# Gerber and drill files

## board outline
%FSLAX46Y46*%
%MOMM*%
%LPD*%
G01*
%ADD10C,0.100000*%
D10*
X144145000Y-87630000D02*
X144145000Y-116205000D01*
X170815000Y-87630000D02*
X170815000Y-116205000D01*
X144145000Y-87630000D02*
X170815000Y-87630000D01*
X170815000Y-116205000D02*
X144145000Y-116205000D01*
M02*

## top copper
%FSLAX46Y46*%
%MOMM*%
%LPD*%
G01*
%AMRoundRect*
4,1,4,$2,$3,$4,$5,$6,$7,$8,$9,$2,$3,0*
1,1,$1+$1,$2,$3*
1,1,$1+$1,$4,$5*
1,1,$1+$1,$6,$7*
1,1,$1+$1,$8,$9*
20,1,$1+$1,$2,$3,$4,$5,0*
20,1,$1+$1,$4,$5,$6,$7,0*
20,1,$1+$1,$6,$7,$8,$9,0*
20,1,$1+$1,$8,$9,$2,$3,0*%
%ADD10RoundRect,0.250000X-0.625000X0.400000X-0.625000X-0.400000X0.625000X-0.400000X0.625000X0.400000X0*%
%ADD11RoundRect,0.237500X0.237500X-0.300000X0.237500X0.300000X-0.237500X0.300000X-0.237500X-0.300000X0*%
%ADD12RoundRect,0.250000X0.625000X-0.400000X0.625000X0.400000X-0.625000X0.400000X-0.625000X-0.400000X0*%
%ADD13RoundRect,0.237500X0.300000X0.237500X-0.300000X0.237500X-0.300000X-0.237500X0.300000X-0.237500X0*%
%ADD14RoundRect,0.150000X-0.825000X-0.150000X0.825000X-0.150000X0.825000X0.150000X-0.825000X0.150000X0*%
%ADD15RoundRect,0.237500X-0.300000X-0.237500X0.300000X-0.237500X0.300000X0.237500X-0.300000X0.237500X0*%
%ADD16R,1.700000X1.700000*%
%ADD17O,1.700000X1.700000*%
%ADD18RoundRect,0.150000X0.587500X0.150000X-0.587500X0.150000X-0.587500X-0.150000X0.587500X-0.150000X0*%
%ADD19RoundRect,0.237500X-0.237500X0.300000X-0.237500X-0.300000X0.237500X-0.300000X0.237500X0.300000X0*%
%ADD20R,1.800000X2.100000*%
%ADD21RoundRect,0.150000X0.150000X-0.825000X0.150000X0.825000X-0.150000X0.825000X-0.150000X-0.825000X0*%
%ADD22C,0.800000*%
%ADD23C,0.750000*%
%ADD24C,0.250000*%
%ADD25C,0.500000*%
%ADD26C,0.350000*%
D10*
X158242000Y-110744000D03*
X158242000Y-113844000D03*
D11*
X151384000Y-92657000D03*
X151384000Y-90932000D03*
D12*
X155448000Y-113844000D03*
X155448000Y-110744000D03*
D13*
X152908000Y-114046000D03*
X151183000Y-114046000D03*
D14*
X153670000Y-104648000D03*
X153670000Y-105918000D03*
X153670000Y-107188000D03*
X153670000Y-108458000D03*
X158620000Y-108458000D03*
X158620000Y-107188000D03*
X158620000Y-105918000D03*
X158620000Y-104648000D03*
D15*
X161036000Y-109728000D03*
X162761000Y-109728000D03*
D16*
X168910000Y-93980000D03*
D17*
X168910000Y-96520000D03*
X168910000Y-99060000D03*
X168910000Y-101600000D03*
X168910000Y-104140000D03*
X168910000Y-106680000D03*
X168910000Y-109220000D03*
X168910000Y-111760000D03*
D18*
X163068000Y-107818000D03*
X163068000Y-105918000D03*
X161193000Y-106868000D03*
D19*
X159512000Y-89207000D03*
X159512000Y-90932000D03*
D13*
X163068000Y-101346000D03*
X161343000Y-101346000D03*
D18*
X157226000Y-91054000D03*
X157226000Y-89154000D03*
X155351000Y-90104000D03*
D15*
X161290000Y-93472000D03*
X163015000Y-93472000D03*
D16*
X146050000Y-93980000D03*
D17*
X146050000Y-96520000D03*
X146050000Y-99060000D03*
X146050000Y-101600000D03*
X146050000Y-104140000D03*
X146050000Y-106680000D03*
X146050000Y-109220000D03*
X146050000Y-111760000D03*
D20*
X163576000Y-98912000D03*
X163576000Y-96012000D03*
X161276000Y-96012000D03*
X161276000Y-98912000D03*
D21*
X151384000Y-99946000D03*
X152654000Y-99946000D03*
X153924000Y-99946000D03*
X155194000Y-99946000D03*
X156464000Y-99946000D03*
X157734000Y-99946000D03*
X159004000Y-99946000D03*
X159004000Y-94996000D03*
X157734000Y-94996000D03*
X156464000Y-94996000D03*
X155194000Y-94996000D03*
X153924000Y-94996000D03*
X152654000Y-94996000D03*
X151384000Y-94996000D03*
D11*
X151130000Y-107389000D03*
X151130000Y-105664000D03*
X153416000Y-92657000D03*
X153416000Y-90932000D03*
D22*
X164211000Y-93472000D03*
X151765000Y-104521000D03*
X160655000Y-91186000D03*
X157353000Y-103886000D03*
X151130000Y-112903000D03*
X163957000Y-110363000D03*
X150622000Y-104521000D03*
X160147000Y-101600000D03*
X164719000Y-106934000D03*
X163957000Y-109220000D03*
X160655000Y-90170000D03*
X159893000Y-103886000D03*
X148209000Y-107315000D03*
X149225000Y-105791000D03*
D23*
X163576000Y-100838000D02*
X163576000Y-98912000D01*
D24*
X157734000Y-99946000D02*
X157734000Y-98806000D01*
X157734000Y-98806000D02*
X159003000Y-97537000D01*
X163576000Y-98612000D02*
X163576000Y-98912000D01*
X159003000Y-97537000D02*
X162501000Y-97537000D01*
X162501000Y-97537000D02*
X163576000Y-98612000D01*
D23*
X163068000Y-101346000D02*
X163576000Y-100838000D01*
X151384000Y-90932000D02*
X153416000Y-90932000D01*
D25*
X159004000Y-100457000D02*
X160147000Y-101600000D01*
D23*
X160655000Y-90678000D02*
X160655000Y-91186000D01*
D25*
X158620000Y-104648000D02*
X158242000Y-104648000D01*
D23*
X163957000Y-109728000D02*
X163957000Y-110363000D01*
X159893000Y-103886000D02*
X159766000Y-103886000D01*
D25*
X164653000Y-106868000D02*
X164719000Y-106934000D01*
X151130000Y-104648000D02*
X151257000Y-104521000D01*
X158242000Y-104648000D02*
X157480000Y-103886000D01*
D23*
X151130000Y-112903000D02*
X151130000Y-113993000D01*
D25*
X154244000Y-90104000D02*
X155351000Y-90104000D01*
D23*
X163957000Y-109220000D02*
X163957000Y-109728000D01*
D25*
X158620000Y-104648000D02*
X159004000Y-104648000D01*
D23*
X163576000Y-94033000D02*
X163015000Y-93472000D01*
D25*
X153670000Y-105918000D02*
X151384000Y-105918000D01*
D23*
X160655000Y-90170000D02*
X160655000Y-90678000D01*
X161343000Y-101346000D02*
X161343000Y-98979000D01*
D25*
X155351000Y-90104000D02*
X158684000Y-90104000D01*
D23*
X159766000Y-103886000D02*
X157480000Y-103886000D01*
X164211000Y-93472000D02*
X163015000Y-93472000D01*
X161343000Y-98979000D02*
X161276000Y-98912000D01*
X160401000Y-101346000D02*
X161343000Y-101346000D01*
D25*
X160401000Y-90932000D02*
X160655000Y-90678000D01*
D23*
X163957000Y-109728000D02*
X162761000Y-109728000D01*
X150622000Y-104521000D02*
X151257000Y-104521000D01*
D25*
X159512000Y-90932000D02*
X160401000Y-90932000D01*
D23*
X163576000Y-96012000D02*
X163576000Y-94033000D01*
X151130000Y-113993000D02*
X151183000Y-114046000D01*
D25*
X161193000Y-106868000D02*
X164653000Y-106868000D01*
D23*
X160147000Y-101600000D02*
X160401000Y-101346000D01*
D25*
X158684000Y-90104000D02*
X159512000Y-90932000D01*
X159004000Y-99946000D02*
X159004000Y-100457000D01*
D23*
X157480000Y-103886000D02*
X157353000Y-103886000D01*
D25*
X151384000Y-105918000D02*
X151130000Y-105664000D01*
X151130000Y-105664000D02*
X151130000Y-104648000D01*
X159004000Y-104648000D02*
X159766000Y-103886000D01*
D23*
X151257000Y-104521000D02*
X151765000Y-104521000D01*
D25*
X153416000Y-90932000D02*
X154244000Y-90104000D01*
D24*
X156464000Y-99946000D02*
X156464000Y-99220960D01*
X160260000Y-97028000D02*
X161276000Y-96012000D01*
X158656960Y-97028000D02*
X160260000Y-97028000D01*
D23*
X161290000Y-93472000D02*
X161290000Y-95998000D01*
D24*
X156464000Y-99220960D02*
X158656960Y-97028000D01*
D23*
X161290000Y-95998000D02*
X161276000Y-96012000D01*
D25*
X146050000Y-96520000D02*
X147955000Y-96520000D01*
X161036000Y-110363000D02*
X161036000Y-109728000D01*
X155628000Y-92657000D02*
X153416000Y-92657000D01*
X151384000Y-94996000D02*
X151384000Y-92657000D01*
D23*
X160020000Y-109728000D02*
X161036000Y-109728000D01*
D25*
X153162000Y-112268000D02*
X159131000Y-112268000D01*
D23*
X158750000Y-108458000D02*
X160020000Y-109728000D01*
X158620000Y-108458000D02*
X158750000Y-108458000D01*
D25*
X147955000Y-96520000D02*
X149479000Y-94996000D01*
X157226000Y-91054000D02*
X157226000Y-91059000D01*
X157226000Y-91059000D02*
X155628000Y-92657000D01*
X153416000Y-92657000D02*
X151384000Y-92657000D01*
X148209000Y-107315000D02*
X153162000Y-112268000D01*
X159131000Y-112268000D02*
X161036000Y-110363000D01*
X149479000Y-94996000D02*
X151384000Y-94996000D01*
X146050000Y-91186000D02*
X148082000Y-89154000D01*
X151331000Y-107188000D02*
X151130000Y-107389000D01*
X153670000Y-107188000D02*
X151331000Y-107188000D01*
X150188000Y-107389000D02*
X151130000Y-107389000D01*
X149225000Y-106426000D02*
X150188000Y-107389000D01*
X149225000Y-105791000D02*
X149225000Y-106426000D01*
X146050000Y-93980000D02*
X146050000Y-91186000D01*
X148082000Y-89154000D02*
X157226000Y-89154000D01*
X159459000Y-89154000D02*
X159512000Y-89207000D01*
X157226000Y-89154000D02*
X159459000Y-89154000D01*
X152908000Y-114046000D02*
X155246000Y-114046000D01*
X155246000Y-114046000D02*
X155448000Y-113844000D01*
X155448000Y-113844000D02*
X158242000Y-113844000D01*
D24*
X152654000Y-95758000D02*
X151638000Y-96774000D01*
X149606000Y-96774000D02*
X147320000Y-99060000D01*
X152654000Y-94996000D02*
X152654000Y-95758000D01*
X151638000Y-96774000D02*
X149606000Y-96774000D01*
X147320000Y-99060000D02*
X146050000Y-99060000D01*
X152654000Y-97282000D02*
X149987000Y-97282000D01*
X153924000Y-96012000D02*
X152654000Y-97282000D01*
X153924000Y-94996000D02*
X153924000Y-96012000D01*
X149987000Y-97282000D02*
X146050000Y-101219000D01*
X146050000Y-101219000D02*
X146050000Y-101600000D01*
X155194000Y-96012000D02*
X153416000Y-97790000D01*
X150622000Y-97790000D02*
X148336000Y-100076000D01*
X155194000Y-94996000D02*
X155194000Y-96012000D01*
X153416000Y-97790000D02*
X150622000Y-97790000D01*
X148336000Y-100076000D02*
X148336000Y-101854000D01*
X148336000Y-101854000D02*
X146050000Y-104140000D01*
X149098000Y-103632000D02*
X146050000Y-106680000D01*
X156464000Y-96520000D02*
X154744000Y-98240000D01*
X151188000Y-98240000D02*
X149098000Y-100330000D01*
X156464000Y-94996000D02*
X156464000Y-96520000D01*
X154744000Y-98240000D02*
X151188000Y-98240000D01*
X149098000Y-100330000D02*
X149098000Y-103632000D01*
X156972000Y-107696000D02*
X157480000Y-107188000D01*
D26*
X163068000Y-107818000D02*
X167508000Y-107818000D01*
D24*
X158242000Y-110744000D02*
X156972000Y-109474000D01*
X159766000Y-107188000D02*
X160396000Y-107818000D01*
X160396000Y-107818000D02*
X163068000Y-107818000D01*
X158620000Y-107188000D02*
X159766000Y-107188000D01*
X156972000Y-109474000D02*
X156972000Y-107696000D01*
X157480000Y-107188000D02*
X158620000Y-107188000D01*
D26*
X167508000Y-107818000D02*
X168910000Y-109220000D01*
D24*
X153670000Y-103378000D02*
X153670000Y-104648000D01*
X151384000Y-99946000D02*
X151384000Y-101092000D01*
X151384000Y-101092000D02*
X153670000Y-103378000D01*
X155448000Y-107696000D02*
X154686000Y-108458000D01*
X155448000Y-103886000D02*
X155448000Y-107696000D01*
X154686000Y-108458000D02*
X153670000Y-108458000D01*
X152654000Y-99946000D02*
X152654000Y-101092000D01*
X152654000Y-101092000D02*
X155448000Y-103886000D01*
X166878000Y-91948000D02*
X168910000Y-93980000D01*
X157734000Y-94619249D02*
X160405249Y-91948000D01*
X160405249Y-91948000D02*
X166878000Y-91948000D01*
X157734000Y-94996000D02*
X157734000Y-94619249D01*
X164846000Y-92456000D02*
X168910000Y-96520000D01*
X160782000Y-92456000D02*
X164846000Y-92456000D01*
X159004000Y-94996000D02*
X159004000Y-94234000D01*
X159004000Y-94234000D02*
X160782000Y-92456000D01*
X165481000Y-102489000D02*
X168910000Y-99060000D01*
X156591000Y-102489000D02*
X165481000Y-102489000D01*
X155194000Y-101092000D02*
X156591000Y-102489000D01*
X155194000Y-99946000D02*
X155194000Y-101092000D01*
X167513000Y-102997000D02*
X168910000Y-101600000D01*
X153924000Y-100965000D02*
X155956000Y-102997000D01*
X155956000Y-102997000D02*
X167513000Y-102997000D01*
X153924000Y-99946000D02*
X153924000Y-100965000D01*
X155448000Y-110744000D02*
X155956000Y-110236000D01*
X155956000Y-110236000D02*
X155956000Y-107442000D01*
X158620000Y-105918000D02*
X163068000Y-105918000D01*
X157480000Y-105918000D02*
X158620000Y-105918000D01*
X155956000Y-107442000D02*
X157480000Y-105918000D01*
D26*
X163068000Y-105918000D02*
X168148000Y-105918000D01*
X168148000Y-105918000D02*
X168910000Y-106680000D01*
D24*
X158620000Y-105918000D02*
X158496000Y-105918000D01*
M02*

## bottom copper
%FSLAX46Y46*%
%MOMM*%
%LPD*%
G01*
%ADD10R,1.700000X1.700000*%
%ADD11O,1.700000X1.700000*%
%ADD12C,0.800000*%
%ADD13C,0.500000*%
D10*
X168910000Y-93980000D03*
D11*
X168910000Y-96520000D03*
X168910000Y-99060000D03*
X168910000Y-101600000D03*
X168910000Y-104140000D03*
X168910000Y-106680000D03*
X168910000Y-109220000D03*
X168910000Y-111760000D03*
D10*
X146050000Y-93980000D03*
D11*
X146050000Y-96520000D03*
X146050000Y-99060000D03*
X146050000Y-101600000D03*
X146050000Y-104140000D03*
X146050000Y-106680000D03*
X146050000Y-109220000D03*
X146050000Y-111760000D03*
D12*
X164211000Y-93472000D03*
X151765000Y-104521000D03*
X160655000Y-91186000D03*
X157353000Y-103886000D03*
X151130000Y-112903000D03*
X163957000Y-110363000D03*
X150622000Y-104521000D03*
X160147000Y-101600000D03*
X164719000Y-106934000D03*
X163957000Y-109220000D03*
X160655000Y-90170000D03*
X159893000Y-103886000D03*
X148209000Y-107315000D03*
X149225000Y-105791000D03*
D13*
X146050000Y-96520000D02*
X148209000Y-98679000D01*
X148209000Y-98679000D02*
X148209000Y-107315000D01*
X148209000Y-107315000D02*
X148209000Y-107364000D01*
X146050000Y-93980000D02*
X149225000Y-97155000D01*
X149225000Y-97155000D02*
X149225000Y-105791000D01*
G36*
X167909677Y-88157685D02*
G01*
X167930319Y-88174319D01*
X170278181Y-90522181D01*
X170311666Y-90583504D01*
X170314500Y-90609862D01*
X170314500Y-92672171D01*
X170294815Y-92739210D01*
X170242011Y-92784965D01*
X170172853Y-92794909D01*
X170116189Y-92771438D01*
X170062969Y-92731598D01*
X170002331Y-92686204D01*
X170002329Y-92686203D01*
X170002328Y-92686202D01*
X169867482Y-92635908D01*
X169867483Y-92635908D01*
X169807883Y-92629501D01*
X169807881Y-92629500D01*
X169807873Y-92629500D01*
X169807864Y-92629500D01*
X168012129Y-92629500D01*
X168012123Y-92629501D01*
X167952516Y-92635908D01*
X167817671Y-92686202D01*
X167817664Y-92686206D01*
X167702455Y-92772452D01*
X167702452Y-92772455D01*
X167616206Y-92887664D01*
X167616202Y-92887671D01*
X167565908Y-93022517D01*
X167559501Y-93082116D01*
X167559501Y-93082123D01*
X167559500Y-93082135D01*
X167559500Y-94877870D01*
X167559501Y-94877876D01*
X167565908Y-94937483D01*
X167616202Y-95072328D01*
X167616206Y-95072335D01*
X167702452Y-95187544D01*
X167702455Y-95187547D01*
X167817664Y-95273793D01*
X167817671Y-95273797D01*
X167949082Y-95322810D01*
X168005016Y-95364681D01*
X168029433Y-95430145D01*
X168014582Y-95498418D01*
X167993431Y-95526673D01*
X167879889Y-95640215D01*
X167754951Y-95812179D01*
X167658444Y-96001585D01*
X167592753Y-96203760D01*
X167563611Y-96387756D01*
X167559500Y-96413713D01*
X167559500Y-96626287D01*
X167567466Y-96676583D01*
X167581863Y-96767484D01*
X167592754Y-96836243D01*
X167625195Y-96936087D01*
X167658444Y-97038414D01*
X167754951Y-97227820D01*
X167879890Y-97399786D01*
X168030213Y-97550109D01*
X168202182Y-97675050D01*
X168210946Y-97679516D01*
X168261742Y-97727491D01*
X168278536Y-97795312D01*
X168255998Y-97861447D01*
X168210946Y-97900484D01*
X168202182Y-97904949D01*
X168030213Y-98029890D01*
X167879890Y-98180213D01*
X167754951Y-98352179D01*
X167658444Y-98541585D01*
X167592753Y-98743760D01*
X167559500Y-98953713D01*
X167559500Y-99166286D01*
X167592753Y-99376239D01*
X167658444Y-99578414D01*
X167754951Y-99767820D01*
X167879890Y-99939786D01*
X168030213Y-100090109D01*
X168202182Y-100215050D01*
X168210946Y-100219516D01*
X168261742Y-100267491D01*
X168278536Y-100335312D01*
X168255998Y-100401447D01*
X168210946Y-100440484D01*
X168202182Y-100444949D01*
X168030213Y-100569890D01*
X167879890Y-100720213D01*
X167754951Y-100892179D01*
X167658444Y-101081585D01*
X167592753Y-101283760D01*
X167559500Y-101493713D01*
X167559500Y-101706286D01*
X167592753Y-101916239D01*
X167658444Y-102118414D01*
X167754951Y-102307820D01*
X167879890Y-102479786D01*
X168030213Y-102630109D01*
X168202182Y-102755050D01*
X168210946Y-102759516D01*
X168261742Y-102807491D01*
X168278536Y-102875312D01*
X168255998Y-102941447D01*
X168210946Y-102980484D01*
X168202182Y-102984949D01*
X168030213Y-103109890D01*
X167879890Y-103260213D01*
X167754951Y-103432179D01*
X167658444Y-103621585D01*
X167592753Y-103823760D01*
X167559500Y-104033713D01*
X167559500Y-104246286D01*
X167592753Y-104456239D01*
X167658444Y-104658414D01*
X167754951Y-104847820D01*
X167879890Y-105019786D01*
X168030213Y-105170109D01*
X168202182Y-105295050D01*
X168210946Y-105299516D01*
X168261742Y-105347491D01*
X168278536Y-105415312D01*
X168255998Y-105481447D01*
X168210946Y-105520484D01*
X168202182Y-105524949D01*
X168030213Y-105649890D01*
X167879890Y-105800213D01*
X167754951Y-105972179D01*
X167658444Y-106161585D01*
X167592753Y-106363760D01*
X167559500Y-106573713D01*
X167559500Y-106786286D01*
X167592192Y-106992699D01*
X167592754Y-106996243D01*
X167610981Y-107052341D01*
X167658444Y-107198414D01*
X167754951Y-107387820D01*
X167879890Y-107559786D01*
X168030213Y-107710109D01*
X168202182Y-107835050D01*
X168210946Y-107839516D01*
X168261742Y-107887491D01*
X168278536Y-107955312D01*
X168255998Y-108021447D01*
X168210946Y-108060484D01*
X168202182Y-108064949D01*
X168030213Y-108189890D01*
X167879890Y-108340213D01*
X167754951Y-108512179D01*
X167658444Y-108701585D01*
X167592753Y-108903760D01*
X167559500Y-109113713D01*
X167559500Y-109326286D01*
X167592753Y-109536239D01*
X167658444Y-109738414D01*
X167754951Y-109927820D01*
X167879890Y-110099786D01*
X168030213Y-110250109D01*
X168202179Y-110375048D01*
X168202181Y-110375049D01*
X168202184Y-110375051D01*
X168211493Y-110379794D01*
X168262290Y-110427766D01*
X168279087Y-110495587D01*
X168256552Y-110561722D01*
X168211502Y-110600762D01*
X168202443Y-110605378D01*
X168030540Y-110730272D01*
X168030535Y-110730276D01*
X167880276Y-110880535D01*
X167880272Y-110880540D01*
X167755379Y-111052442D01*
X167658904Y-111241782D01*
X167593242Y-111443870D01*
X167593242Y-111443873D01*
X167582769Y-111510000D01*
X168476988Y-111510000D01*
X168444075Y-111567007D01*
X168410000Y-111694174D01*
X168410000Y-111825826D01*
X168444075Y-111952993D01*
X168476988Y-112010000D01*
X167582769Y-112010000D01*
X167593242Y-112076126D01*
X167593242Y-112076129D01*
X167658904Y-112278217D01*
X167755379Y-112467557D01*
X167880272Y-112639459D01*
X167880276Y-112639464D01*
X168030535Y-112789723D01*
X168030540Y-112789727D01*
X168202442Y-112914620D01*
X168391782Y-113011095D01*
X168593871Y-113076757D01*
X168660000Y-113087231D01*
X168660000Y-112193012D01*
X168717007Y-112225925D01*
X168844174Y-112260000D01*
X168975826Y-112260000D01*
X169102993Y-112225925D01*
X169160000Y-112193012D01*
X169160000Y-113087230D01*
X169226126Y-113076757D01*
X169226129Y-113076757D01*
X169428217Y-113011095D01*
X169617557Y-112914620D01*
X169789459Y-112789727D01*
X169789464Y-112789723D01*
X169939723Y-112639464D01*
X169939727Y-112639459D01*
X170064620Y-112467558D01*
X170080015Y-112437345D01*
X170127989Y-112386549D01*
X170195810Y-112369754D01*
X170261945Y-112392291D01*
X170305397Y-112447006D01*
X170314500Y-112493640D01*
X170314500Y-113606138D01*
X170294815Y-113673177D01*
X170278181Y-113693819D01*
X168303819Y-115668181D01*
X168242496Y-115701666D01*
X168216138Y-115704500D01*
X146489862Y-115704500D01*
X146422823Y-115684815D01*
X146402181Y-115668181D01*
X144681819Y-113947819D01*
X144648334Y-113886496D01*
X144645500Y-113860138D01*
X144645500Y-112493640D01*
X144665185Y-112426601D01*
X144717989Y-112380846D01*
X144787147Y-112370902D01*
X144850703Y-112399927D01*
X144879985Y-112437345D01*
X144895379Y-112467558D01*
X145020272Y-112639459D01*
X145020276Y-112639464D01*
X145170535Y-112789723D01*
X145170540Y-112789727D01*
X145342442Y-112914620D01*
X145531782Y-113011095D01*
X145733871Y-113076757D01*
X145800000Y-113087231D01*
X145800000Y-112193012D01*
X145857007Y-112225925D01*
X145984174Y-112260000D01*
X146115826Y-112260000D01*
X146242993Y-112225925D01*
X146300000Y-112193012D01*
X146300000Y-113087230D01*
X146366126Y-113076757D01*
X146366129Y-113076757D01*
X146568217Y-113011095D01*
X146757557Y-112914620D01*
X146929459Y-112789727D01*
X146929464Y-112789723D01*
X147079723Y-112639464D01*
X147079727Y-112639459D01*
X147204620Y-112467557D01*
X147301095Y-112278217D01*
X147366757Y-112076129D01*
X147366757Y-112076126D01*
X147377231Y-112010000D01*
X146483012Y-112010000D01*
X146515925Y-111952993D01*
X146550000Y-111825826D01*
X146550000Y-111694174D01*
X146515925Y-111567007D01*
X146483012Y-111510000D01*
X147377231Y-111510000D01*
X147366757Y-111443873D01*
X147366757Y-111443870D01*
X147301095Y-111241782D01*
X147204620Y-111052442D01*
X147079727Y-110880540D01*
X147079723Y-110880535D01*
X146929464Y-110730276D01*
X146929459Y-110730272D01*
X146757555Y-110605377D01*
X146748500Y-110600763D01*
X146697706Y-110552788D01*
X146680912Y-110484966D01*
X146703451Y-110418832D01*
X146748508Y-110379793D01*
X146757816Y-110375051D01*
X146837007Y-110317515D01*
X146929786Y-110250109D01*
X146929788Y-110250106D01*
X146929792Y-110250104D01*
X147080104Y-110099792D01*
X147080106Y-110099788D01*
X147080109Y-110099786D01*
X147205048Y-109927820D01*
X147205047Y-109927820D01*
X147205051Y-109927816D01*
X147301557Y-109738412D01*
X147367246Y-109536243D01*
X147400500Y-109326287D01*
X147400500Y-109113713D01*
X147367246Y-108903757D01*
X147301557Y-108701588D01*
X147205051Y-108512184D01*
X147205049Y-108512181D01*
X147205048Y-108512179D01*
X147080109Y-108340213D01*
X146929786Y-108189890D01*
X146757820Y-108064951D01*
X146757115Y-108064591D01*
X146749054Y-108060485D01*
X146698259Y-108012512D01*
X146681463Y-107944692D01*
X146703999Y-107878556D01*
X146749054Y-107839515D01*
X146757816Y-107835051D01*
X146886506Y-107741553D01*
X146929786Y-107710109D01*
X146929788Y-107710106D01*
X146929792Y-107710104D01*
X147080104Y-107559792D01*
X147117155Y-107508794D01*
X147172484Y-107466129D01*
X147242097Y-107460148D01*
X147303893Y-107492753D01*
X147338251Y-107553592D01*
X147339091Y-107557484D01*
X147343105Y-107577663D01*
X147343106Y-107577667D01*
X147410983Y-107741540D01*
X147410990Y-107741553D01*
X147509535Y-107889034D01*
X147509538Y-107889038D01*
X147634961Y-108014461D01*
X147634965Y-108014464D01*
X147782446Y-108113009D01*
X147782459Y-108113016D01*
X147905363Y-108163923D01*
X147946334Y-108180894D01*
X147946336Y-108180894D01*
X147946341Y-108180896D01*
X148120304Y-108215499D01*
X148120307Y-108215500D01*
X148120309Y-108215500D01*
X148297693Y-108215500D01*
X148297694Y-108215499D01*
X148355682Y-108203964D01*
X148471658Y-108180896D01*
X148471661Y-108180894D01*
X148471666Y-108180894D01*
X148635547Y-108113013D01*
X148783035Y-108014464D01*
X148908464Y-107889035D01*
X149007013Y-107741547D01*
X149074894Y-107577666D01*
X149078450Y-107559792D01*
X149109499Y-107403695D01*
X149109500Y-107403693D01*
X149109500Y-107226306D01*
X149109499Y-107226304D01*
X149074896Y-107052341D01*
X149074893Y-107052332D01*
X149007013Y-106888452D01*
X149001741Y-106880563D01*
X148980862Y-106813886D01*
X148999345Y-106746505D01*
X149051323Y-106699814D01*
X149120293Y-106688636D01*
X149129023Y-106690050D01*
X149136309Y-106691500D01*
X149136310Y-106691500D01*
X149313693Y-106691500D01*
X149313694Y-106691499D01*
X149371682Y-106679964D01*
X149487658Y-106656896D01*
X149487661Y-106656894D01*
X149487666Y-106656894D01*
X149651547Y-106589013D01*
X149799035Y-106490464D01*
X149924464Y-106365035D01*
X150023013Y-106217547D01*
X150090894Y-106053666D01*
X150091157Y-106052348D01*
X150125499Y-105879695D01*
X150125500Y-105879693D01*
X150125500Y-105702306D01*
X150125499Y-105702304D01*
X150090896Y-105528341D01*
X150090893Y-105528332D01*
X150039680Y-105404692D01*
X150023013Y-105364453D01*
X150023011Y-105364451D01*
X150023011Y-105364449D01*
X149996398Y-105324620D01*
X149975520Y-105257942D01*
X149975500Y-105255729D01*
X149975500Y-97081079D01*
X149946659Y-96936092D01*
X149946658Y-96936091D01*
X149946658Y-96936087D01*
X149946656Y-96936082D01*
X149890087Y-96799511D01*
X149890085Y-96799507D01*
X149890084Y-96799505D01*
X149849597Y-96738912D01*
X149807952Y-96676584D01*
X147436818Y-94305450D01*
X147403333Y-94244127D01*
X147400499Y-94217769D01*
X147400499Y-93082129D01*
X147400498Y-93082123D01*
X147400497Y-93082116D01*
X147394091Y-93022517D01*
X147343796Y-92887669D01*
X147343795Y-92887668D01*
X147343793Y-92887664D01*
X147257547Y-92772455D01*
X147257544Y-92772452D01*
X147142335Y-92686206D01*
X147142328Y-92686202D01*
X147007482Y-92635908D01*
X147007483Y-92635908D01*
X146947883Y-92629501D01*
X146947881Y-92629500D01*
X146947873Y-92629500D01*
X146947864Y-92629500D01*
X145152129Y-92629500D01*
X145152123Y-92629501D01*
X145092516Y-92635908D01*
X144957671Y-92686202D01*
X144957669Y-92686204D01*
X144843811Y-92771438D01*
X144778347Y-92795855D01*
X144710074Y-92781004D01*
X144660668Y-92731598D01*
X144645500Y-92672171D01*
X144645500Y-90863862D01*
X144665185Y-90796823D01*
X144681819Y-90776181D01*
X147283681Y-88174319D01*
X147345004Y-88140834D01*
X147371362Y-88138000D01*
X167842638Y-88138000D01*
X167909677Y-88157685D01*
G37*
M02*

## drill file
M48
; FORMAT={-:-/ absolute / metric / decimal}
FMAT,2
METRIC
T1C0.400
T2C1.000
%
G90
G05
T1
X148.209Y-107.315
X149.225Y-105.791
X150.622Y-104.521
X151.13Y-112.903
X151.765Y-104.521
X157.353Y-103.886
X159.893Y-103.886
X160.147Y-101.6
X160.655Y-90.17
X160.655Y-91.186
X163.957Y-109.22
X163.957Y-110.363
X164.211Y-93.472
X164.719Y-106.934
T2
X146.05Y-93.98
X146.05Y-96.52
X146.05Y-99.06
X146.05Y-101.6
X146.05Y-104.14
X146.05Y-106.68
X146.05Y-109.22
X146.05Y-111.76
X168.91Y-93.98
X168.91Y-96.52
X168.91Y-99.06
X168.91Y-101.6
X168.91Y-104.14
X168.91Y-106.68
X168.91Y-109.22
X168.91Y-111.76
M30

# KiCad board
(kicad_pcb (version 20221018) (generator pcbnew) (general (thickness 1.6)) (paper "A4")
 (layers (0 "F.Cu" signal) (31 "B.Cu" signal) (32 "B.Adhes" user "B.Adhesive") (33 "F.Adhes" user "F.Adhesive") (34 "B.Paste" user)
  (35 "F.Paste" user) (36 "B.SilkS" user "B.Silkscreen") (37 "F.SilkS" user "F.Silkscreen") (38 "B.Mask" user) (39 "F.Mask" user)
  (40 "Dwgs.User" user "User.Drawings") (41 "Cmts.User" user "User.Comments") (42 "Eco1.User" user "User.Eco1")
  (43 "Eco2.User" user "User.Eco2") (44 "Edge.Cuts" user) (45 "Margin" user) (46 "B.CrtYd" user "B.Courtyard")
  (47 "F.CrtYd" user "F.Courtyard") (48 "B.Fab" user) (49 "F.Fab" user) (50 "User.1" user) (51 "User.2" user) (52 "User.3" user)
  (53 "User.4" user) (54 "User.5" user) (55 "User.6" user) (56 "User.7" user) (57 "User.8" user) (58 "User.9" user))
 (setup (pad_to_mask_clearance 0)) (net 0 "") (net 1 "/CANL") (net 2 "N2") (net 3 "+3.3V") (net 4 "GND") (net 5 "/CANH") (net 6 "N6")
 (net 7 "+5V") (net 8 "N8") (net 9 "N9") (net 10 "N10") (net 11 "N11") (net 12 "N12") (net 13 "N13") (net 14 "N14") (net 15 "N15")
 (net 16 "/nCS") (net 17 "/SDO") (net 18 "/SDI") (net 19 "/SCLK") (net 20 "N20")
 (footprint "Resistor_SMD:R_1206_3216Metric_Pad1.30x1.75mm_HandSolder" (layer "F.Cu") (at 158.242 112.294 -90)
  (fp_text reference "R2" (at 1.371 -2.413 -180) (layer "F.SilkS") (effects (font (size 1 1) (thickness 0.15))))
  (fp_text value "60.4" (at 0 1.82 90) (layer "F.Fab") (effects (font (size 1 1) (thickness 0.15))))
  (pad "1" smd roundrect (at -1.55 0 270) (size 1.3 1.75) (layers "F.Cu" "F.Paste" "F.Mask") (roundrect_rratio 0.1923076923) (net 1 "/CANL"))
  (pad "2" smd roundrect (at 1.55 0 270) (size 1.3 1.75) (layers "F.Cu" "F.Paste" "F.Mask") (roundrect_rratio 0.1923076923) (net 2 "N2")))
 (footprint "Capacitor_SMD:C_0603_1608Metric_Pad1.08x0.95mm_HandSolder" (layer "F.Cu") (at 151.384 91.7945 90)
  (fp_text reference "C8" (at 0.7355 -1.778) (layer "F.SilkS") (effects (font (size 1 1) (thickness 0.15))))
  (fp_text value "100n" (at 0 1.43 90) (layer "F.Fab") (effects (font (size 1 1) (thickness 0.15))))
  (pad "1" smd roundrect (at -0.8625 0 90) (size 1.075 0.95) (layers "F.Cu" "F.Paste" "F.Mask") (roundrect_rratio 0.25) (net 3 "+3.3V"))
  (pad "2" smd roundrect (at 0.8625 0 90) (size 1.075 0.95) (layers "F.Cu" "F.Paste" "F.Mask") (roundrect_rratio 0.25) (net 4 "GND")))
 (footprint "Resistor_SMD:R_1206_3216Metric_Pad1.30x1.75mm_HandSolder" (layer "F.Cu") (at 155.448 112.294 90)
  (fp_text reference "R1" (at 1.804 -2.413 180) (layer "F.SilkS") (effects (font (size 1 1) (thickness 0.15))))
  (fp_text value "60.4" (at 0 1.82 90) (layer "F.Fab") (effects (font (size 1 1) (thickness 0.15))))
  (pad "1" smd roundrect (at -1.55 0 90) (size 1.3 1.75) (layers "F.Cu" "F.Paste" "F.Mask") (roundrect_rratio 0.1923076923) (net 2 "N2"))
  (pad "2" smd roundrect (at 1.55 0 90) (size 1.3 1.75) (layers "F.Cu" "F.Paste" "F.Mask") (roundrect_rratio 0.1923076923) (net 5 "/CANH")))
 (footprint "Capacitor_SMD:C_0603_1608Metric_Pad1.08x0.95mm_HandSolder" (layer "F.Cu") (at 152.0455 114.046 180)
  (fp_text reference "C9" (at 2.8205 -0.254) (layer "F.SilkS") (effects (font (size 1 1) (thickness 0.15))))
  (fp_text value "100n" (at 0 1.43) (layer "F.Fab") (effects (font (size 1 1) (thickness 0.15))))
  (pad "1" smd roundrect (at -0.8625 0 180) (size 1.075 0.95) (layers "F.Cu" "F.Paste" "F.Mask") (roundrect_rratio 0.25) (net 2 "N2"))
  (pad "2" smd roundrect (at 0.8625 0 180) (size 1.075 0.95) (layers "F.Cu" "F.Paste" "F.Mask") (roundrect_rratio 0.25) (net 4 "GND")))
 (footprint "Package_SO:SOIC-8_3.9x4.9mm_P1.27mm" (layer "F.Cu") (at 156.145 106.553)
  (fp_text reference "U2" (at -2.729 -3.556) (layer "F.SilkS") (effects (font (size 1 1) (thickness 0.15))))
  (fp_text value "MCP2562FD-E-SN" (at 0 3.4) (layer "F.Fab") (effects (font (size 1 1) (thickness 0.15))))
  (pad "1" smd roundrect (at -2.475 -1.905) (size 1.95 0.6) (layers "F.Cu" "F.Paste" "F.Mask") (roundrect_rratio 0.25) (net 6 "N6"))
  (pad "2" smd roundrect (at -2.475 -0.635) (size 1.95 0.6) (layers "F.Cu" "F.Paste" "F.Mask") (roundrect_rratio 0.25) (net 4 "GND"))
  (pad "3" smd roundrect (at -2.475 0.635) (size 1.95 0.6) (layers "F.Cu" "F.Paste" "F.Mask") (roundrect_rratio 0.25) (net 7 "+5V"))
  (pad "4" smd roundrect (at -2.475 1.905) (size 1.95 0.6) (layers "F.Cu" "F.Paste" "F.Mask") (roundrect_rratio 0.25) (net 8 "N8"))
  (pad "5" smd roundrect (at 2.475 1.905) (size 1.95 0.6) (layers "F.Cu" "F.Paste" "F.Mask") (roundrect_rratio 0.25) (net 3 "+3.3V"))
  (pad "6" smd roundrect (at 2.475 0.635) (size 1.95 0.6) (layers "F.Cu" "F.Paste" "F.Mask") (roundrect_rratio 0.25) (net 1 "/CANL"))
  (pad "7" smd roundrect (at 2.475 -0.635) (size 1.95 0.6) (layers "F.Cu" "F.Paste" "F.Mask") (roundrect_rratio 0.25) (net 5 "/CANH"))
  (pad "8" smd roundrect (at 2.475 -1.905) (size 1.95 0.6) (layers "F.Cu" "F.Paste" "F.Mask") (roundrect_rratio 0.25) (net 4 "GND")))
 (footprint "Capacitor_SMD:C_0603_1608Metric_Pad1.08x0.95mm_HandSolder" (layer "F.Cu") (at 161.8985 109.728)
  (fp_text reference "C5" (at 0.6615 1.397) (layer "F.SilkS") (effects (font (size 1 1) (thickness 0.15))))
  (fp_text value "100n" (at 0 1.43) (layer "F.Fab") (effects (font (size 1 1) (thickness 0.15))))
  (pad "1" smd roundrect (at -0.8625 0) (size 1.075 0.95) (layers "F.Cu" "F.Paste" "F.Mask") (roundrect_rratio 0.25) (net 3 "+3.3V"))
  (pad "2" smd roundrect (at 0.8625 0) (size 1.075 0.95) (layers "F.Cu" "F.Paste" "F.Mask") (roundrect_rratio 0.25) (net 4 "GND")))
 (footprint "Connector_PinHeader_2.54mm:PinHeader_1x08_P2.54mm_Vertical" (layer "F.Cu") (at 168.91 93.98)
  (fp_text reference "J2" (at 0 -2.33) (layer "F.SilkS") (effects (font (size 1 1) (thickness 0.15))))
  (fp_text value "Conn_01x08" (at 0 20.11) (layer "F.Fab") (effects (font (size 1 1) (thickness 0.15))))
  (pad "1" thru_hole rect (at 0 0) (size 1.7 1.7) (drill 1) (layers "*.Cu" "*.Mask") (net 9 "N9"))
  (pad "2" thru_hole oval (at 0 2.54) (size 1.7 1.7) (drill 1) (layers "*.Cu" "*.Mask") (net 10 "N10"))
  (pad "3" thru_hole oval (at 0 5.08) (size 1.7 1.7) (drill 1) (layers "*.Cu" "*.Mask") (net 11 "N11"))
  (pad "4" thru_hole oval (at 0 7.62) (size 1.7 1.7) (drill 1) (layers "*.Cu" "*.Mask") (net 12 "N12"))
  (pad "5" thru_hole oval (at 0 10.16) (size 1.7 1.7) (drill 1) (layers "*.Cu" "*.Mask") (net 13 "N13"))
  (pad "6" thru_hole oval (at 0 12.7) (size 1.7 1.7) (drill 1) (layers "*.Cu" "*.Mask") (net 5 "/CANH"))
  (pad "7" thru_hole oval (at 0 15.24) (size 1.7 1.7) (drill 1) (layers "*.Cu" "*.Mask") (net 1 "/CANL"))
  (pad "8" thru_hole oval (at 0 17.78) (size 1.7 1.7) (drill 1) (layers "*.Cu" "*.Mask") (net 4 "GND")))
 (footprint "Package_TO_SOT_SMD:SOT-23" (layer "F.Cu") (at 162.1305 106.868 180)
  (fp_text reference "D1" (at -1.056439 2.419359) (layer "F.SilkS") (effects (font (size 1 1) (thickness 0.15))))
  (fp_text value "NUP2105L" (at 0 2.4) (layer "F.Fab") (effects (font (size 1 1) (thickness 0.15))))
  (pad "1" smd roundrect (at -0.9375 -0.95 180) (size 1.475 0.6) (layers "F.Cu" "F.Paste" "F.Mask") (roundrect_rratio 0.25) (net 1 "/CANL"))
  (pad "2" smd roundrect (at -0.9375 0.95 180) (size 1.475 0.6) (layers "F.Cu" "F.Paste" "F.Mask") (roundrect_rratio 0.25) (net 5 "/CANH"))
  (pad "3" smd roundrect (at 0.9375 0 180) (size 1.475 0.6) (layers "F.Cu" "F.Paste" "F.Mask") (roundrect_rratio 0.25) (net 4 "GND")))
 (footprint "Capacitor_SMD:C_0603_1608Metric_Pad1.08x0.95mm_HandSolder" (layer "F.Cu") (at 159.512 90.0695 -90)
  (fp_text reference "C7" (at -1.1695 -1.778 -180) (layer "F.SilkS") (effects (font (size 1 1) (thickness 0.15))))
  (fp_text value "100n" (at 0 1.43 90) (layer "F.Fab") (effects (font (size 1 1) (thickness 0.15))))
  (pad "1" smd roundrect (at -0.8625 0 270) (size 1.075 0.95) (layers "F.Cu" "F.Paste" "F.Mask") (roundrect_rratio 0.25) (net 7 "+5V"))
  (pad "2" smd roundrect (at 0.8625 0 270) (size 1.075 0.95) (layers "F.Cu" "F.Paste" "F.Mask") (roundrect_rratio 0.25) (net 4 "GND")))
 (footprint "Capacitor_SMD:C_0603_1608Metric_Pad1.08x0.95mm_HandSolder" (layer "F.Cu") (at 162.2055 101.346 180)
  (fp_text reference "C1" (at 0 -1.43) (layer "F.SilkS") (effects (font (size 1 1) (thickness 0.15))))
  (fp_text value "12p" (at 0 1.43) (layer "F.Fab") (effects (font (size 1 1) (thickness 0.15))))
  (pad "1" smd roundrect (at -0.8625 0 180) (size 1.075 0.95) (layers "F.Cu" "F.Paste" "F.Mask") (roundrect_rratio 0.25) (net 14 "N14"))
  (pad "2" smd roundrect (at 0.8625 0 180) (size 1.075 0.95) (layers "F.Cu" "F.Paste" "F.Mask") (roundrect_rratio 0.25) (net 4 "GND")))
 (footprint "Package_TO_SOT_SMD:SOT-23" (layer "F.Cu") (at 156.2885 90.104 180)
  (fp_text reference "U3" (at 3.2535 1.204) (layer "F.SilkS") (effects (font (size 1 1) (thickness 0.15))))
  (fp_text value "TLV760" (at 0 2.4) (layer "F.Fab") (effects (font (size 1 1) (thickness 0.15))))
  (pad "1" smd roundrect (at -0.9375 -0.95 180) (size 1.475 0.6) (layers "F.Cu" "F.Paste" "F.Mask") (roundrect_rratio 0.25) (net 3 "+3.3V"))
  (pad "2" smd roundrect (at -0.9375 0.95 180) (size 1.475 0.6) (layers "F.Cu" "F.Paste" "F.Mask") (roundrect_rratio 0.25) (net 7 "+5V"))
  (pad "3" smd roundrect (at 0.9375 0 180) (size 1.475 0.6) (layers "F.Cu" "F.Paste" "F.Mask") (roundrect_rratio 0.25) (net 4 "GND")))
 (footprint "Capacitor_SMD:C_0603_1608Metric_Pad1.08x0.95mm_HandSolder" (layer "F.Cu") (at 162.1525 93.472)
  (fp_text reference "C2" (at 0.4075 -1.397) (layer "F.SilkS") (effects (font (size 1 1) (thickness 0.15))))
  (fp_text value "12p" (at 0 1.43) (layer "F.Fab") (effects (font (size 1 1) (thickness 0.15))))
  (pad "1" smd roundrect (at -0.8625 0) (size 1.075 0.95) (layers "F.Cu" "F.Paste" "F.Mask") (roundrect_rratio 0.25) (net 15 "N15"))
  (pad "2" smd roundrect (at 0.8625 0) (size 1.075 0.95) (layers "F.Cu" "F.Paste" "F.Mask") (roundrect_rratio 0.25) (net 4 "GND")))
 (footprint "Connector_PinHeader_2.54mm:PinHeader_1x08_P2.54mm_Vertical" (layer "F.Cu") (at 146.05 93.98)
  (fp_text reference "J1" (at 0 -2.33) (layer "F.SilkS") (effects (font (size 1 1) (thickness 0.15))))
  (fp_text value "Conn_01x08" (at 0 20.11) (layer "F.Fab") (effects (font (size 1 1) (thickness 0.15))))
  (pad "1" thru_hole rect (at 0 0) (size 1.7 1.7) (drill 1) (layers "*.Cu" "*.Mask") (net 7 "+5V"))
  (pad "2" thru_hole oval (at 0 2.54) (size 1.7 1.7) (drill 1) (layers "*.Cu" "*.Mask") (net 3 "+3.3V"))
  (pad "3" thru_hole oval (at 0 5.08) (size 1.7 1.7) (drill 1) (layers "*.Cu" "*.Mask") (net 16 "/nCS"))
  (pad "4" thru_hole oval (at 0 7.62) (size 1.7 1.7) (drill 1) (layers "*.Cu" "*.Mask") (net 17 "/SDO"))
  (pad "5" thru_hole oval (at 0 10.16) (size 1.7 1.7) (drill 1) (layers "*.Cu" "*.Mask") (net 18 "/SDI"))
  (pad "6" thru_hole oval (at 0 12.7) (size 1.7 1.7) (drill 1) (layers "*.Cu" "*.Mask") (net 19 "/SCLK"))
  (pad "7" thru_hole oval (at 0 15.24) (size 1.7 1.7) (drill 1) (layers "*.Cu" "*.Mask") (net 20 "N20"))
  (pad "8" thru_hole oval (at 0 17.78) (size 1.7 1.7) (drill 1) (layers "*.Cu" "*.Mask") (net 4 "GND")))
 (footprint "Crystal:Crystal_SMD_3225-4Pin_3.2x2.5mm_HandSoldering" (layer "F.Cu") (at 162.426 97.462 90)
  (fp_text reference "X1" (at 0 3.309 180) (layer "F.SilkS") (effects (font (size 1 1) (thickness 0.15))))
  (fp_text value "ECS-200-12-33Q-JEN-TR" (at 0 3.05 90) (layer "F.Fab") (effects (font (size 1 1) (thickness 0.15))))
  (pad "1" smd rect (at -1.45 1.15 90) (size 2.1 1.8) (layers "F.Cu" "F.Paste" "F.Mask") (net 14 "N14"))
  (pad "2" smd rect (at 1.45 1.15 90) (size 2.1 1.8) (layers "F.Cu" "F.Paste" "F.Mask") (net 4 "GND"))
  (pad "3" smd rect (at 1.45 -1.15 90) (size 2.1 1.8) (layers "F.Cu" "F.Paste" "F.Mask") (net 15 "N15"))
  (pad "4" smd rect (at -1.45 -1.15 90) (size 2.1 1.8) (layers "F.Cu" "F.Paste" "F.Mask") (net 4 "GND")))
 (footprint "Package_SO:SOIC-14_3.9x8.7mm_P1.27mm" (layer "F.Cu") (at 155.194 97.471 90)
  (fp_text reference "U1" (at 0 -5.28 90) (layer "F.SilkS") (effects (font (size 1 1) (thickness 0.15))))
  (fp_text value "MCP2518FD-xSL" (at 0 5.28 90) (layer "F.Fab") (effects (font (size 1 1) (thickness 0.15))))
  (pad "1" smd roundrect (at -2.475 -3.81 90) (size 1.95 0.6) (layers "F.Cu" "F.Paste" "F.Mask") (roundrect_rratio 0.25) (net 6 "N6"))
  (pad "2" smd roundrect (at -2.475 -2.54 90) (size 1.95 0.6) (layers "F.Cu" "F.Paste" "F.Mask") (roundrect_rratio 0.25) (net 8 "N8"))
  (pad "3" smd roundrect (at -2.475 -1.27 90) (size 1.95 0.6) (layers "F.Cu" "F.Paste" "F.Mask") (roundrect_rratio 0.25) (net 12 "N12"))
  (pad "4" smd roundrect (at -2.475 0 90) (size 1.95 0.6) (layers "F.Cu" "F.Paste" "F.Mask") (roundrect_rratio 0.25) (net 11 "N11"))
  (pad "5" smd roundrect (at -2.475 1.27 90) (size 1.95 0.6) (layers "F.Cu" "F.Paste" "F.Mask") (roundrect_rratio 0.25) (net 15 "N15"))
  (pad "6" smd roundrect (at -2.475 2.54 90) (size 1.95 0.6) (layers "F.Cu" "F.Paste" "F.Mask") (roundrect_rratio 0.25) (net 14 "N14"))
  (pad "7" smd roundrect (at -2.475 3.81 90) (size 1.95 0.6) (layers "F.Cu" "F.Paste" "F.Mask") (roundrect_rratio 0.25) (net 4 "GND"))
  (pad "8" smd roundrect (at 2.475 3.81 90) (size 1.95 0.6) (layers "F.Cu" "F.Paste" "F.Mask") (roundrect_rratio 0.25) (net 10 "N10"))
  (pad "9" smd roundrect (at 2.475 2.54 90) (size 1.95 0.6) (layers "F.Cu" "F.Paste" "F.Mask") (roundrect_rratio 0.25) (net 9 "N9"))
  (pad "10" smd roundrect (at 2.475 1.27 90) (size 1.95 0.6) (layers "F.Cu" "F.Paste" "F.Mask") (roundrect_rratio 0.25) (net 19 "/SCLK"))
  (pad "11" smd roundrect (at 2.475 0 90) (size 1.95 0.6) (layers "F.Cu" "F.Paste" "F.Mask") (roundrect_rratio 0.25) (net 18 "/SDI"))
  (pad "12" smd roundrect (at 2.475 -1.27 90) (size 1.95 0.6) (layers "F.Cu" "F.Paste" "F.Mask") (roundrect_rratio 0.25) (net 17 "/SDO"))
  (pad "13" smd roundrect (at 2.475 -2.54 90) (size 1.95 0.6) (layers "F.Cu" "F.Paste" "F.Mask") (roundrect_rratio 0.25) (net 16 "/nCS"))
  (pad "14" smd roundrect (at 2.475 -3.81 90) (size 1.95 0.6) (layers "F.Cu" "F.Paste" "F.Mask") (roundrect_rratio 0.25) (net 3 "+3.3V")))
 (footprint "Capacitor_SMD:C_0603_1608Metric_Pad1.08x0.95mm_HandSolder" (layer "F.Cu") (at 151.13 106.5265 90)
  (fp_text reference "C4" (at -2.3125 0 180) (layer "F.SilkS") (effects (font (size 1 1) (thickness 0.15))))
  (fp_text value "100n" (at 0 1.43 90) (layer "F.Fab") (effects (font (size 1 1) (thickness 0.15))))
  (pad "1" smd roundrect (at -0.8625 0 90) (size 1.075 0.95) (layers "F.Cu" "F.Paste" "F.Mask") (roundrect_rratio 0.25) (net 7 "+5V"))
  (pad "2" smd roundrect (at 0.8625 0 90) (size 1.075 0.95) (layers "F.Cu" "F.Paste" "F.Mask") (roundrect_rratio 0.25) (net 4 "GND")))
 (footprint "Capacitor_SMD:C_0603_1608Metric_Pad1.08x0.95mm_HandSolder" (layer "F.Cu") (at 153.416 91.7945 90)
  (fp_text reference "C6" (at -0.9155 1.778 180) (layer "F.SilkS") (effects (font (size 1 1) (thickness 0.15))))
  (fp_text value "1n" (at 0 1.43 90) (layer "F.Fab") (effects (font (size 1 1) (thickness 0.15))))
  (pad "1" smd roundrect (at -0.8625 0 90) (size 1.075 0.95) (layers "F.Cu" "F.Paste" "F.Mask") (roundrect_rratio 0.25) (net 3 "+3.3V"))
  (pad "2" smd roundrect (at 0.8625 0 90) (size 1.075 0.95) (layers "F.Cu" "F.Paste" "F.Mask") (roundrect_rratio 0.25) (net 4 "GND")))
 (gr_line (start 144.145 87.63) (end 144.145 116.205) (stroke (width 0.1) (type default)) (layer "Edge.Cuts"))
 (gr_line (start 170.815 87.63) (end 170.815 116.205) (stroke (width 0.1) (type default)) (layer "Edge.Cuts"))
 (gr_line (start 144.145 87.63) (end 170.815 87.63) (stroke (width 0.1) (type default)) (layer "Edge.Cuts"))
 (gr_line (start 170.815 116.205) (end 144.145 116.205) (stroke (width 0.1) (type default)) (layer "Edge.Cuts"))
 (segment (start 163.576 100.838) (end 163.576 98.912) (width 0.75) (layer "F.Cu") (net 14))
 (segment (start 157.734 99.946) (end 157.734 98.806) (width 0.25) (layer "F.Cu") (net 14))
 (segment (start 157.734 98.806) (end 159.003 97.537) (width 0.25) (layer "F.Cu") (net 14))
 (segment (start 163.576 98.612) (end 163.576 98.912) (width 0.25) (layer "F.Cu") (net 14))
 (segment (start 159.003 97.537) (end 162.501 97.537) (width 0.25) (layer "F.Cu") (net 14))
 (segment (start 162.501 97.537) (end 163.576 98.612) (width 0.25) (layer "F.Cu") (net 14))
 (segment (start 163.068 101.346) (end 163.576 100.838) (width 0.75) (layer "F.Cu") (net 14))
 (segment (start 151.384 90.932) (end 153.416 90.932) (width 0.75) (layer "F.Cu") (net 4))
 (segment (start 159.004 100.457) (end 160.147 101.6) (width 0.5) (layer "F.Cu") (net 4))
 (segment (start 160.655 90.678) (end 160.655 91.186) (width 0.75) (layer "F.Cu") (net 4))
 (segment (start 158.62 104.648) (end 158.242 104.648) (width 0.5) (layer "F.Cu") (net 4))
 (segment (start 163.957 109.728) (end 163.957 110.363) (width 0.75) (layer "F.Cu") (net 4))
 (segment (start 159.893 103.886) (end 159.766 103.886) (width 0.75) (layer "F.Cu") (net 4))
 (segment (start 164.653 106.868) (end 164.719 106.934) (width 0.5) (layer "F.Cu") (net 4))
 (segment (start 151.13 104.648) (end 151.257 104.521) (width 0.5) (layer "F.Cu") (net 4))
 (segment (start 158.242 104.648) (end 157.48 103.886) (width 0.5) (layer "F.Cu") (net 4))
 (segment (start 151.13 112.903) (end 151.13 113.993) (width 0.75) (layer "F.Cu") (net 4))
 (segment (start 154.244 90.104) (end 155.351 90.104) (width 0.5) (layer "F.Cu") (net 4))
 (segment (start 163.957 109.22) (end 163.957 109.728) (width 0.75) (layer "F.Cu") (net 4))
 (segment (start 158.62 104.648) (end 159.004 104.648) (width 0.5) (layer "F.Cu") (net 4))
 (segment (start 163.576 94.033) (end 163.015 93.472) (width 0.75) (layer "F.Cu") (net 4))
 (segment (start 153.67 105.918) (end 151.384 105.918) (width 0.5) (layer "F.Cu") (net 4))
 (segment (start 160.655 90.17) (end 160.655 90.678) (width 0.75) (layer "F.Cu") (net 4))
 (segment (start 161.343 101.346) (end 161.343 98.979) (width 0.75) (layer "F.Cu") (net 4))
 (segment (start 155.351 90.104) (end 158.684 90.104) (width 0.5) (layer "F.Cu") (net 4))
 (segment (start 159.766 103.886) (end 157.48 103.886) (width 0.75) (layer "F.Cu") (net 4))
 (segment (start 164.211 93.472) (end 163.015 93.472) (width 0.75) (layer "F.Cu") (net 4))
 (segment (start 161.343 98.979) (end 161.276 98.912) (width 0.75) (layer "F.Cu") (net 4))
 (segment (start 160.401 101.346) (end 161.343 101.346) (width 0.75) (layer "F.Cu") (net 4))
 (segment (start 160.401 90.932) (end 160.655 90.678) (width 0.5) (layer "F.Cu") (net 4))
 (segment (start 163.957 109.728) (end 162.761 109.728) (width 0.75) (layer "F.Cu") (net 4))
 (segment (start 150.622 104.521) (end 151.257 104.521) (width 0.75) (layer "F.Cu") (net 4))
 (segment (start 159.512 90.932) (end 160.401 90.932) (width 0.5) (layer "F.Cu") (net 4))
 (segment (start 163.576 96.012) (end 163.576 94.033) (width 0.75) (layer "F.Cu") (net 4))
 (segment (start 151.13 113.993) (end 151.183 114.046) (width 0.75) (layer "F.Cu") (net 4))
 (segment (start 161.193 106.868) (end 164.653 106.868) (width 0.5) (layer "F.Cu") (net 4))
 (segment (start 160.147 101.6) (end 160.401 101.346) (width 0.75) (layer "F.Cu") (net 4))
 (segment (start 158.684 90.104) (end 159.512 90.932) (width 0.5) (layer "F.Cu") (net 4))
 (segment (start 159.004 99.946) (end 159.004 100.457) (width 0.5) (layer "F.Cu") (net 4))
 (segment (start 157.48 103.886) (end 157.353 103.886) (width 0.75) (layer "F.Cu") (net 4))
 (segment (start 151.384 105.918) (end 151.13 105.664) (width 0.5) (layer "F.Cu") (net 4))
 (segment (start 151.13 105.664) (end 151.13 104.648) (width 0.5) (layer "F.Cu") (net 4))
 (segment (start 159.004 104.648) (end 159.766 103.886) (width 0.5) (layer "F.Cu") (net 4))
 (segment (start 151.257 104.521) (end 151.765 104.521) (width 0.75) (layer "F.Cu") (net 4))
 (segment (start 153.416 90.932) (end 154.244 90.104) (width 0.5) (layer "F.Cu") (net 4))
 (via (at 164.211 93.472) (size 0.8) (drill 0.4) (layers "F.Cu" "B.Cu") (free) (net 4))
 (via (at 151.765 104.521) (size 0.8) (drill 0.4) (layers "F.Cu" "B.Cu") (free) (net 4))
 (via (at 160.655 91.186) (size 0.8) (drill 0.4) (layers "F.Cu" "B.Cu") (free) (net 4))
 (via (at 157.353 103.886) (size 0.8) (drill 0.4) (layers "F.Cu" "B.Cu") (free) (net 4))
 (via (at 151.13 112.903) (size 0.8) (drill 0.4) (layers "F.Cu" "B.Cu") (free) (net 4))
 (via (at 163.957 110.363) (size 0.8) (drill 0.4) (layers "F.Cu" "B.Cu") (free) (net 4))
 (via (at 150.622 104.521) (size 0.8) (drill 0.4) (layers "F.Cu" "B.Cu") (free) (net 4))
 (via (at 160.147 101.6) (size 0.8) (drill 0.4) (layers "F.Cu" "B.Cu") (free) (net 4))
 (via (at 164.719 106.934) (size 0.8) (drill 0.4) (layers "F.Cu" "B.Cu") (free) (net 4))
 (via (at 163.957 109.22) (size 0.8) (drill 0.4) (layers "F.Cu" "B.Cu") (free) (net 4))
 (via (at 160.655 90.17) (size 0.8) (drill 0.4) (layers "F.Cu" "B.Cu") (free) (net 4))
 (via (at 159.893 103.886) (size 0.8) (drill 0.4) (layers "F.Cu" "B.Cu") (free) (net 4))
 (segment (start 156.464 99.946) (end 156.464 99.22096) (width 0.25) (layer "F.Cu") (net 15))
 (segment (start 160.26 97.028) (end 161.276 96.012) (width 0.25) (layer "F.Cu") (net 15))
 (segment (start 158.65696 97.028) (end 160.26 97.028) (width 0.25) (layer "F.Cu") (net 15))
 (segment (start 161.29 93.472) (end 161.29 95.998) (width 0.75) (layer "F.Cu") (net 15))
 (segment (start 156.464 99.22096) (end 158.65696 97.028) (width 0.25) (layer "F.Cu") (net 15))
 (segment (start 161.29 95.998) (end 161.276 96.012) (width 0.75) (layer "F.Cu") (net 15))
 (segment (start 146.05 96.52) (end 147.955 96.52) (width 0.5) (layer "F.Cu") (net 3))
 (segment (start 161.036 110.363) (end 161.036 109.728) (width 0.5) (layer "F.Cu") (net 3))
 (segment (start 155.628 92.657) (end 153.416 92.657) (width 0.5) (layer "F.Cu") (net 3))
 (segment (start 151.384 94.996) (end 151.384 92.657) (width 0.5) (layer "F.Cu") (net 3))
 (segment (start 160.02 109.728) (end 161.036 109.728) (width 0.75) (layer "F.Cu") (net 3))
 (segment (start 153.162 112.268) (end 159.131 112.268) (width 0.5) (layer "F.Cu") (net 3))
 (segment (start 158.75 108.458) (end 160.02 109.728) (width 0.75) (layer "F.Cu") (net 3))
 (segment (start 158.62 108.458) (end 158.75 108.458) (width 0.75) (layer "F.Cu") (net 3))
 (segment (start 147.955 96.52) (end 149.479 94.996) (width 0.5) (layer "F.Cu") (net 3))
 (segment (start 157.226 91.054) (end 157.226 91.059) (width 0.5) (layer "F.Cu") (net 3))
 (segment (start 157.226 91.059) (end 155.628 92.657) (width 0.5) (layer "F.Cu") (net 3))
 (segment (start 153.416 92.657) (end 151.384 92.657) (width 0.5) (layer "F.Cu") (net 3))
 (segment (start 148.209 107.315) (end 153.162 112.268) (width 0.5) (layer "F.Cu") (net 3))
 (segment (start 159.131 112.268) (end 161.036 110.363) (width 0.5) (layer "F.Cu") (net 3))
 (segment (start 149.479 94.996) (end 151.384 94.996) (width 0.5) (layer "F.Cu") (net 3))
 (via (at 148.209 107.315) (size 0.8) (drill 0.4) (layers "F.Cu" "B.Cu") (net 3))
 (segment (start 146.05 96.52) (end 148.209 98.679) (width 0.5) (layer "B.Cu") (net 3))
 (segment (start 148.209 98.679) (end 148.209 107.315) (width 0.5) (layer "B.Cu") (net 3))
 (segment (start 148.209 107.315) (end 148.209 107.364) (width 0.5) (layer "B.Cu") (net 3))
 (segment (start 146.05 91.186) (end 148.082 89.154) (width 0.5) (layer "F.Cu") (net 7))
 (segment (start 151.331 107.188) (end 151.13 107.389) (width 0.5) (layer "F.Cu") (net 7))
 (segment (start 153.67 107.188) (end 151.331 107.188) (width 0.5) (layer "F.Cu") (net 7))
 (segment (start 150.188 107.389) (end 151.13 107.389) (width 0.5) (layer "F.Cu") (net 7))
 (segment (start 149.225 106.426) (end 150.188 107.389) (width 0.5) (layer "F.Cu") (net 7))
 (segment (start 149.225 105.791) (end 149.225 106.426) (width 0.5) (layer "F.Cu") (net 7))
 (segment (start 146.05 93.98) (end 146.05 91.186) (width 0.5) (layer "F.Cu") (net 7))
 (segment (start 148.082 89.154) (end 157.226 89.154) (width 0.5) (layer "F.Cu") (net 7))
 (segment (start 159.459 89.154) (end 159.512 89.207) (width 0.5) (layer "F.Cu") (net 7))
 (segment (start 157.226 89.154) (end 159.459 89.154) (width 0.5) (layer "F.Cu") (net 7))
 (via (at 149.225 105.791) (size 0.8) (drill 0.4) (layers "F.Cu" "B.Cu") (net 7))
 (segment (start 146.05 93.98) (end 149.225 97.155) (width 0.5) (layer "B.Cu") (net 7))
 (segment (start 149.225 97.155) (end 149.225 105.791) (width 0.5) (layer "B.Cu") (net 7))
 (segment (start 152.908 114.046) (end 155.246 114.046) (width 0.5) (layer "F.Cu") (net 2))
 (segment (start 155.246 114.046) (end 155.448 113.844) (width 0.5) (layer "F.Cu") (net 2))
 (segment (start 155.448 113.844) (end 158.242 113.844) (width 0.5) (layer "F.Cu") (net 2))
 (segment (start 152.654 95.758) (end 151.638 96.774) (width 0.25) (layer "F.Cu") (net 16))
 (segment (start 149.606 96.774) (end 147.32 99.06) (width 0.25) (layer "F.Cu") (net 16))
 (segment (start 152.654 94.996) (end 152.654 95.758) (width 0.25) (layer "F.Cu") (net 16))
 (segment (start 151.638 96.774) (end 149.606 96.774) (width 0.25) (layer "F.Cu") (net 16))
 (segment (start 147.32 99.06) (end 146.05 99.06) (width 0.25) (layer "F.Cu") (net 16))
 (segment (start 152.654 97.282) (end 149.987 97.282) (width 0.25) (layer "F.Cu") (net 17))
 (segment (start 153.924 96.012) (end 152.654 97.282) (width 0.25) (layer "F.Cu") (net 17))
 (segment (start 153.924 94.996) (end 153.924 96.012) (width 0.25) (layer "F.Cu") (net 17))
 (segment (start 149.987 97.282) (end 146.05 101.219) (width 0.25) (layer "F.Cu") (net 17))
 (segment (start 146.05 101.219) (end 146.05 101.6) (width 0.25) (layer "F.Cu") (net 17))
 (segment (start 155.194 96.012) (end 153.416 97.79) (width 0.25) (layer "F.Cu") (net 18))
 (segment (start 150.622 97.79) (end 148.336 100.076) (width 0.25) (layer "F.Cu") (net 18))
 (segment (start 155.194 94.996) (end 155.194 96.012) (width 0.25) (layer "F.Cu") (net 18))
 (segment (start 153.416 97.79) (end 150.622 97.79) (width 0.25) (layer "F.Cu") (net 18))
 (segment (start 148.336 100.076) (end 148.336 101.854) (width 0.25) (layer "F.Cu") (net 18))
 (segment (start 148.336 101.854) (end 146.05 104.14) (width 0.25) (layer "F.Cu") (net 18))
 (segment (start 149.098 103.632) (end 146.05 106.68) (width 0.25) (layer "F.Cu") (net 19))
 (segment (start 156.464 96.52) (end 154.744 98.24) (width 0.25) (layer "F.Cu") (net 19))
 (segment (start 151.188 98.24) (end 149.098 100.33) (width 0.25) (layer "F.Cu") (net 19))
 (segment (start 156.464 94.996) (end 156.464 96.52) (width 0.25) (layer "F.Cu") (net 19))
 (segment (start 154.744 98.24) (end 151.188 98.24) (width 0.25) (layer "F.Cu") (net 19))
 (segment (start 149.098 100.33) (end 149.098 103.632) (width 0.25) (layer "F.Cu") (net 19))
 (segment (start 156.972 107.696) (end 157.48 107.188) (width 0.25) (layer "F.Cu") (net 1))
 (segment (start 163.068 107.818) (end 167.508 107.818) (width 0.35) (layer "F.Cu") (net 1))
 (segment (start 158.242 110.744) (end 156.972 109.474) (width 0.25) (layer "F.Cu") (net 1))
 (segment (start 159.766 107.188) (end 160.396 107.818) (width 0.25) (layer "F.Cu") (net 1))
 (segment (start 160.396 107.818) (end 163.068 107.818) (width 0.25) (layer "F.Cu") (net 1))
 (segment (start 158.62 107.188) (end 159.766 107.188) (width 0.25) (layer "F.Cu") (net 1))
 (segment (start 156.972 109.474) (end 156.972 107.696) (width 0.25) (layer "F.Cu") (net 1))
 (segment (start 157.48 107.188) (end 158.62 107.188) (width 0.25) (layer "F.Cu") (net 1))
 (segment (start 167.508 107.818) (end 168.91 109.22) (width 0.35) (layer "F.Cu") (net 1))
 (segment (start 153.67 103.378) (end 153.67 104.648) (width 0.25) (layer "F.Cu") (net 6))
 (segment (start 151.384 99.946) (end 151.384 101.092) (width 0.25) (layer "F.Cu") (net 6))
 (segment (start 151.384 101.092) (end 153.67 103.378) (width 0.25) (layer "F.Cu") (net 6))
 (segment (start 155.448 107.696) (end 154.686 108.458) (width 0.25) (layer "F.Cu") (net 8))
 (segment (start 155.448 103.886) (end 155.448 107.696) (width 0.25) (layer "F.Cu") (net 8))
 (segment (start 154.686 108.458) (end 153.67 108.458) (width 0.25) (layer "F.Cu") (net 8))
 (segment (start 152.654 99.946) (end 152.654 101.092) (width 0.25) (layer "F.Cu") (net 8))
 (segment (start 152.654 101.092) (end 155.448 103.886) (width 0.25) (layer "F.Cu") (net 8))
 (segment (start 166.878 91.948) (end 168.91 93.98) (width 0.25) (layer "F.Cu") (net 9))
 (segment (start 157.734 94.619249) (end 160.405249 91.948) (width 0.25) (layer "F.Cu") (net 9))
 (segment (start 160.405249 91.948) (end 166.878 91.948) (width 0.25) (layer "F.Cu") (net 9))
 (segment (start 157.734 94.996) (end 157.734 94.619249) (width 0.25) (layer "F.Cu") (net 9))
 (segment (start 164.846 92.456) (end 168.91 96.52) (width 0.25) (layer "F.Cu") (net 10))
 (segment (start 160.782 92.456) (end 164.846 92.456) (width 0.25) (layer "F.Cu") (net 10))
 (segment (start 159.004 94.996) (end 159.004 94.234) (width 0.25) (layer "F.Cu") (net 10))
 (segment (start 159.004 94.234) (end 160.782 92.456) (width 0.25) (layer "F.Cu") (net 10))
 (segment (start 165.481 102.489) (end 168.91 99.06) (width 0.25) (layer "F.Cu") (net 11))
 (segment (start 156.591 102.489) (end 165.481 102.489) (width 0.25) (layer "F.Cu") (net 11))
 (segment (start 155.194 101.092) (end 156.591 102.489) (width 0.25) (layer "F.Cu") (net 11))
 (segment (start 155.194 99.946) (end 155.194 101.092) (width 0.25) (layer "F.Cu") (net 11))
 (segment (start 167.513 102.997) (end 168.91 101.6) (width 0.25) (layer "F.Cu") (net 12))
 (segment (start 153.924 100.965) (end 155.956 102.997) (width 0.25) (layer "F.Cu") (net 12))
 (segment (start 155.956 102.997) (end 167.513 102.997) (width 0.25) (layer "F.Cu") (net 12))
 (segment (start 153.924 99.946) (end 153.924 100.965) (width 0.25) (layer "F.Cu") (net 12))
 (segment (start 155.448 110.744) (end 155.956 110.236) (width 0.25) (layer "F.Cu") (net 5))
 (segment (start 155.956 110.236) (end 155.956 107.442) (width 0.25) (layer "F.Cu") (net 5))
 (segment (start 158.62 105.918) (end 163.068 105.918) (width 0.25) (layer "F.Cu") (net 5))
 (segment (start 157.48 105.918) (end 158.62 105.918) (width 0.25) (layer "F.Cu") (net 5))
 (segment (start 155.956 107.442) (end 157.48 105.918) (width 0.25) (layer "F.Cu") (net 5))
 (segment (start 163.068 105.918) (end 168.148 105.918) (width 0.35) (layer "F.Cu") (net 5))
 (segment (start 168.148 105.918) (end 168.91 106.68) (width 0.35) (layer "F.Cu") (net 5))
 (segment (start 158.62 105.918) (end 158.496 105.918) (width 0.25) (layer "F.Cu") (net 5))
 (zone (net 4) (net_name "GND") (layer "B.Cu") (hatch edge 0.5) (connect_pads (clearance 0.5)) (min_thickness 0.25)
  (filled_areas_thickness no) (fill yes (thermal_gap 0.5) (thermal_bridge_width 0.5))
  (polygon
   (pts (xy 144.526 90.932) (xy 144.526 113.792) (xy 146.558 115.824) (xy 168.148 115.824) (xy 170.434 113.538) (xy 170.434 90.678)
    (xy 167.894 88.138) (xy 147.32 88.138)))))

